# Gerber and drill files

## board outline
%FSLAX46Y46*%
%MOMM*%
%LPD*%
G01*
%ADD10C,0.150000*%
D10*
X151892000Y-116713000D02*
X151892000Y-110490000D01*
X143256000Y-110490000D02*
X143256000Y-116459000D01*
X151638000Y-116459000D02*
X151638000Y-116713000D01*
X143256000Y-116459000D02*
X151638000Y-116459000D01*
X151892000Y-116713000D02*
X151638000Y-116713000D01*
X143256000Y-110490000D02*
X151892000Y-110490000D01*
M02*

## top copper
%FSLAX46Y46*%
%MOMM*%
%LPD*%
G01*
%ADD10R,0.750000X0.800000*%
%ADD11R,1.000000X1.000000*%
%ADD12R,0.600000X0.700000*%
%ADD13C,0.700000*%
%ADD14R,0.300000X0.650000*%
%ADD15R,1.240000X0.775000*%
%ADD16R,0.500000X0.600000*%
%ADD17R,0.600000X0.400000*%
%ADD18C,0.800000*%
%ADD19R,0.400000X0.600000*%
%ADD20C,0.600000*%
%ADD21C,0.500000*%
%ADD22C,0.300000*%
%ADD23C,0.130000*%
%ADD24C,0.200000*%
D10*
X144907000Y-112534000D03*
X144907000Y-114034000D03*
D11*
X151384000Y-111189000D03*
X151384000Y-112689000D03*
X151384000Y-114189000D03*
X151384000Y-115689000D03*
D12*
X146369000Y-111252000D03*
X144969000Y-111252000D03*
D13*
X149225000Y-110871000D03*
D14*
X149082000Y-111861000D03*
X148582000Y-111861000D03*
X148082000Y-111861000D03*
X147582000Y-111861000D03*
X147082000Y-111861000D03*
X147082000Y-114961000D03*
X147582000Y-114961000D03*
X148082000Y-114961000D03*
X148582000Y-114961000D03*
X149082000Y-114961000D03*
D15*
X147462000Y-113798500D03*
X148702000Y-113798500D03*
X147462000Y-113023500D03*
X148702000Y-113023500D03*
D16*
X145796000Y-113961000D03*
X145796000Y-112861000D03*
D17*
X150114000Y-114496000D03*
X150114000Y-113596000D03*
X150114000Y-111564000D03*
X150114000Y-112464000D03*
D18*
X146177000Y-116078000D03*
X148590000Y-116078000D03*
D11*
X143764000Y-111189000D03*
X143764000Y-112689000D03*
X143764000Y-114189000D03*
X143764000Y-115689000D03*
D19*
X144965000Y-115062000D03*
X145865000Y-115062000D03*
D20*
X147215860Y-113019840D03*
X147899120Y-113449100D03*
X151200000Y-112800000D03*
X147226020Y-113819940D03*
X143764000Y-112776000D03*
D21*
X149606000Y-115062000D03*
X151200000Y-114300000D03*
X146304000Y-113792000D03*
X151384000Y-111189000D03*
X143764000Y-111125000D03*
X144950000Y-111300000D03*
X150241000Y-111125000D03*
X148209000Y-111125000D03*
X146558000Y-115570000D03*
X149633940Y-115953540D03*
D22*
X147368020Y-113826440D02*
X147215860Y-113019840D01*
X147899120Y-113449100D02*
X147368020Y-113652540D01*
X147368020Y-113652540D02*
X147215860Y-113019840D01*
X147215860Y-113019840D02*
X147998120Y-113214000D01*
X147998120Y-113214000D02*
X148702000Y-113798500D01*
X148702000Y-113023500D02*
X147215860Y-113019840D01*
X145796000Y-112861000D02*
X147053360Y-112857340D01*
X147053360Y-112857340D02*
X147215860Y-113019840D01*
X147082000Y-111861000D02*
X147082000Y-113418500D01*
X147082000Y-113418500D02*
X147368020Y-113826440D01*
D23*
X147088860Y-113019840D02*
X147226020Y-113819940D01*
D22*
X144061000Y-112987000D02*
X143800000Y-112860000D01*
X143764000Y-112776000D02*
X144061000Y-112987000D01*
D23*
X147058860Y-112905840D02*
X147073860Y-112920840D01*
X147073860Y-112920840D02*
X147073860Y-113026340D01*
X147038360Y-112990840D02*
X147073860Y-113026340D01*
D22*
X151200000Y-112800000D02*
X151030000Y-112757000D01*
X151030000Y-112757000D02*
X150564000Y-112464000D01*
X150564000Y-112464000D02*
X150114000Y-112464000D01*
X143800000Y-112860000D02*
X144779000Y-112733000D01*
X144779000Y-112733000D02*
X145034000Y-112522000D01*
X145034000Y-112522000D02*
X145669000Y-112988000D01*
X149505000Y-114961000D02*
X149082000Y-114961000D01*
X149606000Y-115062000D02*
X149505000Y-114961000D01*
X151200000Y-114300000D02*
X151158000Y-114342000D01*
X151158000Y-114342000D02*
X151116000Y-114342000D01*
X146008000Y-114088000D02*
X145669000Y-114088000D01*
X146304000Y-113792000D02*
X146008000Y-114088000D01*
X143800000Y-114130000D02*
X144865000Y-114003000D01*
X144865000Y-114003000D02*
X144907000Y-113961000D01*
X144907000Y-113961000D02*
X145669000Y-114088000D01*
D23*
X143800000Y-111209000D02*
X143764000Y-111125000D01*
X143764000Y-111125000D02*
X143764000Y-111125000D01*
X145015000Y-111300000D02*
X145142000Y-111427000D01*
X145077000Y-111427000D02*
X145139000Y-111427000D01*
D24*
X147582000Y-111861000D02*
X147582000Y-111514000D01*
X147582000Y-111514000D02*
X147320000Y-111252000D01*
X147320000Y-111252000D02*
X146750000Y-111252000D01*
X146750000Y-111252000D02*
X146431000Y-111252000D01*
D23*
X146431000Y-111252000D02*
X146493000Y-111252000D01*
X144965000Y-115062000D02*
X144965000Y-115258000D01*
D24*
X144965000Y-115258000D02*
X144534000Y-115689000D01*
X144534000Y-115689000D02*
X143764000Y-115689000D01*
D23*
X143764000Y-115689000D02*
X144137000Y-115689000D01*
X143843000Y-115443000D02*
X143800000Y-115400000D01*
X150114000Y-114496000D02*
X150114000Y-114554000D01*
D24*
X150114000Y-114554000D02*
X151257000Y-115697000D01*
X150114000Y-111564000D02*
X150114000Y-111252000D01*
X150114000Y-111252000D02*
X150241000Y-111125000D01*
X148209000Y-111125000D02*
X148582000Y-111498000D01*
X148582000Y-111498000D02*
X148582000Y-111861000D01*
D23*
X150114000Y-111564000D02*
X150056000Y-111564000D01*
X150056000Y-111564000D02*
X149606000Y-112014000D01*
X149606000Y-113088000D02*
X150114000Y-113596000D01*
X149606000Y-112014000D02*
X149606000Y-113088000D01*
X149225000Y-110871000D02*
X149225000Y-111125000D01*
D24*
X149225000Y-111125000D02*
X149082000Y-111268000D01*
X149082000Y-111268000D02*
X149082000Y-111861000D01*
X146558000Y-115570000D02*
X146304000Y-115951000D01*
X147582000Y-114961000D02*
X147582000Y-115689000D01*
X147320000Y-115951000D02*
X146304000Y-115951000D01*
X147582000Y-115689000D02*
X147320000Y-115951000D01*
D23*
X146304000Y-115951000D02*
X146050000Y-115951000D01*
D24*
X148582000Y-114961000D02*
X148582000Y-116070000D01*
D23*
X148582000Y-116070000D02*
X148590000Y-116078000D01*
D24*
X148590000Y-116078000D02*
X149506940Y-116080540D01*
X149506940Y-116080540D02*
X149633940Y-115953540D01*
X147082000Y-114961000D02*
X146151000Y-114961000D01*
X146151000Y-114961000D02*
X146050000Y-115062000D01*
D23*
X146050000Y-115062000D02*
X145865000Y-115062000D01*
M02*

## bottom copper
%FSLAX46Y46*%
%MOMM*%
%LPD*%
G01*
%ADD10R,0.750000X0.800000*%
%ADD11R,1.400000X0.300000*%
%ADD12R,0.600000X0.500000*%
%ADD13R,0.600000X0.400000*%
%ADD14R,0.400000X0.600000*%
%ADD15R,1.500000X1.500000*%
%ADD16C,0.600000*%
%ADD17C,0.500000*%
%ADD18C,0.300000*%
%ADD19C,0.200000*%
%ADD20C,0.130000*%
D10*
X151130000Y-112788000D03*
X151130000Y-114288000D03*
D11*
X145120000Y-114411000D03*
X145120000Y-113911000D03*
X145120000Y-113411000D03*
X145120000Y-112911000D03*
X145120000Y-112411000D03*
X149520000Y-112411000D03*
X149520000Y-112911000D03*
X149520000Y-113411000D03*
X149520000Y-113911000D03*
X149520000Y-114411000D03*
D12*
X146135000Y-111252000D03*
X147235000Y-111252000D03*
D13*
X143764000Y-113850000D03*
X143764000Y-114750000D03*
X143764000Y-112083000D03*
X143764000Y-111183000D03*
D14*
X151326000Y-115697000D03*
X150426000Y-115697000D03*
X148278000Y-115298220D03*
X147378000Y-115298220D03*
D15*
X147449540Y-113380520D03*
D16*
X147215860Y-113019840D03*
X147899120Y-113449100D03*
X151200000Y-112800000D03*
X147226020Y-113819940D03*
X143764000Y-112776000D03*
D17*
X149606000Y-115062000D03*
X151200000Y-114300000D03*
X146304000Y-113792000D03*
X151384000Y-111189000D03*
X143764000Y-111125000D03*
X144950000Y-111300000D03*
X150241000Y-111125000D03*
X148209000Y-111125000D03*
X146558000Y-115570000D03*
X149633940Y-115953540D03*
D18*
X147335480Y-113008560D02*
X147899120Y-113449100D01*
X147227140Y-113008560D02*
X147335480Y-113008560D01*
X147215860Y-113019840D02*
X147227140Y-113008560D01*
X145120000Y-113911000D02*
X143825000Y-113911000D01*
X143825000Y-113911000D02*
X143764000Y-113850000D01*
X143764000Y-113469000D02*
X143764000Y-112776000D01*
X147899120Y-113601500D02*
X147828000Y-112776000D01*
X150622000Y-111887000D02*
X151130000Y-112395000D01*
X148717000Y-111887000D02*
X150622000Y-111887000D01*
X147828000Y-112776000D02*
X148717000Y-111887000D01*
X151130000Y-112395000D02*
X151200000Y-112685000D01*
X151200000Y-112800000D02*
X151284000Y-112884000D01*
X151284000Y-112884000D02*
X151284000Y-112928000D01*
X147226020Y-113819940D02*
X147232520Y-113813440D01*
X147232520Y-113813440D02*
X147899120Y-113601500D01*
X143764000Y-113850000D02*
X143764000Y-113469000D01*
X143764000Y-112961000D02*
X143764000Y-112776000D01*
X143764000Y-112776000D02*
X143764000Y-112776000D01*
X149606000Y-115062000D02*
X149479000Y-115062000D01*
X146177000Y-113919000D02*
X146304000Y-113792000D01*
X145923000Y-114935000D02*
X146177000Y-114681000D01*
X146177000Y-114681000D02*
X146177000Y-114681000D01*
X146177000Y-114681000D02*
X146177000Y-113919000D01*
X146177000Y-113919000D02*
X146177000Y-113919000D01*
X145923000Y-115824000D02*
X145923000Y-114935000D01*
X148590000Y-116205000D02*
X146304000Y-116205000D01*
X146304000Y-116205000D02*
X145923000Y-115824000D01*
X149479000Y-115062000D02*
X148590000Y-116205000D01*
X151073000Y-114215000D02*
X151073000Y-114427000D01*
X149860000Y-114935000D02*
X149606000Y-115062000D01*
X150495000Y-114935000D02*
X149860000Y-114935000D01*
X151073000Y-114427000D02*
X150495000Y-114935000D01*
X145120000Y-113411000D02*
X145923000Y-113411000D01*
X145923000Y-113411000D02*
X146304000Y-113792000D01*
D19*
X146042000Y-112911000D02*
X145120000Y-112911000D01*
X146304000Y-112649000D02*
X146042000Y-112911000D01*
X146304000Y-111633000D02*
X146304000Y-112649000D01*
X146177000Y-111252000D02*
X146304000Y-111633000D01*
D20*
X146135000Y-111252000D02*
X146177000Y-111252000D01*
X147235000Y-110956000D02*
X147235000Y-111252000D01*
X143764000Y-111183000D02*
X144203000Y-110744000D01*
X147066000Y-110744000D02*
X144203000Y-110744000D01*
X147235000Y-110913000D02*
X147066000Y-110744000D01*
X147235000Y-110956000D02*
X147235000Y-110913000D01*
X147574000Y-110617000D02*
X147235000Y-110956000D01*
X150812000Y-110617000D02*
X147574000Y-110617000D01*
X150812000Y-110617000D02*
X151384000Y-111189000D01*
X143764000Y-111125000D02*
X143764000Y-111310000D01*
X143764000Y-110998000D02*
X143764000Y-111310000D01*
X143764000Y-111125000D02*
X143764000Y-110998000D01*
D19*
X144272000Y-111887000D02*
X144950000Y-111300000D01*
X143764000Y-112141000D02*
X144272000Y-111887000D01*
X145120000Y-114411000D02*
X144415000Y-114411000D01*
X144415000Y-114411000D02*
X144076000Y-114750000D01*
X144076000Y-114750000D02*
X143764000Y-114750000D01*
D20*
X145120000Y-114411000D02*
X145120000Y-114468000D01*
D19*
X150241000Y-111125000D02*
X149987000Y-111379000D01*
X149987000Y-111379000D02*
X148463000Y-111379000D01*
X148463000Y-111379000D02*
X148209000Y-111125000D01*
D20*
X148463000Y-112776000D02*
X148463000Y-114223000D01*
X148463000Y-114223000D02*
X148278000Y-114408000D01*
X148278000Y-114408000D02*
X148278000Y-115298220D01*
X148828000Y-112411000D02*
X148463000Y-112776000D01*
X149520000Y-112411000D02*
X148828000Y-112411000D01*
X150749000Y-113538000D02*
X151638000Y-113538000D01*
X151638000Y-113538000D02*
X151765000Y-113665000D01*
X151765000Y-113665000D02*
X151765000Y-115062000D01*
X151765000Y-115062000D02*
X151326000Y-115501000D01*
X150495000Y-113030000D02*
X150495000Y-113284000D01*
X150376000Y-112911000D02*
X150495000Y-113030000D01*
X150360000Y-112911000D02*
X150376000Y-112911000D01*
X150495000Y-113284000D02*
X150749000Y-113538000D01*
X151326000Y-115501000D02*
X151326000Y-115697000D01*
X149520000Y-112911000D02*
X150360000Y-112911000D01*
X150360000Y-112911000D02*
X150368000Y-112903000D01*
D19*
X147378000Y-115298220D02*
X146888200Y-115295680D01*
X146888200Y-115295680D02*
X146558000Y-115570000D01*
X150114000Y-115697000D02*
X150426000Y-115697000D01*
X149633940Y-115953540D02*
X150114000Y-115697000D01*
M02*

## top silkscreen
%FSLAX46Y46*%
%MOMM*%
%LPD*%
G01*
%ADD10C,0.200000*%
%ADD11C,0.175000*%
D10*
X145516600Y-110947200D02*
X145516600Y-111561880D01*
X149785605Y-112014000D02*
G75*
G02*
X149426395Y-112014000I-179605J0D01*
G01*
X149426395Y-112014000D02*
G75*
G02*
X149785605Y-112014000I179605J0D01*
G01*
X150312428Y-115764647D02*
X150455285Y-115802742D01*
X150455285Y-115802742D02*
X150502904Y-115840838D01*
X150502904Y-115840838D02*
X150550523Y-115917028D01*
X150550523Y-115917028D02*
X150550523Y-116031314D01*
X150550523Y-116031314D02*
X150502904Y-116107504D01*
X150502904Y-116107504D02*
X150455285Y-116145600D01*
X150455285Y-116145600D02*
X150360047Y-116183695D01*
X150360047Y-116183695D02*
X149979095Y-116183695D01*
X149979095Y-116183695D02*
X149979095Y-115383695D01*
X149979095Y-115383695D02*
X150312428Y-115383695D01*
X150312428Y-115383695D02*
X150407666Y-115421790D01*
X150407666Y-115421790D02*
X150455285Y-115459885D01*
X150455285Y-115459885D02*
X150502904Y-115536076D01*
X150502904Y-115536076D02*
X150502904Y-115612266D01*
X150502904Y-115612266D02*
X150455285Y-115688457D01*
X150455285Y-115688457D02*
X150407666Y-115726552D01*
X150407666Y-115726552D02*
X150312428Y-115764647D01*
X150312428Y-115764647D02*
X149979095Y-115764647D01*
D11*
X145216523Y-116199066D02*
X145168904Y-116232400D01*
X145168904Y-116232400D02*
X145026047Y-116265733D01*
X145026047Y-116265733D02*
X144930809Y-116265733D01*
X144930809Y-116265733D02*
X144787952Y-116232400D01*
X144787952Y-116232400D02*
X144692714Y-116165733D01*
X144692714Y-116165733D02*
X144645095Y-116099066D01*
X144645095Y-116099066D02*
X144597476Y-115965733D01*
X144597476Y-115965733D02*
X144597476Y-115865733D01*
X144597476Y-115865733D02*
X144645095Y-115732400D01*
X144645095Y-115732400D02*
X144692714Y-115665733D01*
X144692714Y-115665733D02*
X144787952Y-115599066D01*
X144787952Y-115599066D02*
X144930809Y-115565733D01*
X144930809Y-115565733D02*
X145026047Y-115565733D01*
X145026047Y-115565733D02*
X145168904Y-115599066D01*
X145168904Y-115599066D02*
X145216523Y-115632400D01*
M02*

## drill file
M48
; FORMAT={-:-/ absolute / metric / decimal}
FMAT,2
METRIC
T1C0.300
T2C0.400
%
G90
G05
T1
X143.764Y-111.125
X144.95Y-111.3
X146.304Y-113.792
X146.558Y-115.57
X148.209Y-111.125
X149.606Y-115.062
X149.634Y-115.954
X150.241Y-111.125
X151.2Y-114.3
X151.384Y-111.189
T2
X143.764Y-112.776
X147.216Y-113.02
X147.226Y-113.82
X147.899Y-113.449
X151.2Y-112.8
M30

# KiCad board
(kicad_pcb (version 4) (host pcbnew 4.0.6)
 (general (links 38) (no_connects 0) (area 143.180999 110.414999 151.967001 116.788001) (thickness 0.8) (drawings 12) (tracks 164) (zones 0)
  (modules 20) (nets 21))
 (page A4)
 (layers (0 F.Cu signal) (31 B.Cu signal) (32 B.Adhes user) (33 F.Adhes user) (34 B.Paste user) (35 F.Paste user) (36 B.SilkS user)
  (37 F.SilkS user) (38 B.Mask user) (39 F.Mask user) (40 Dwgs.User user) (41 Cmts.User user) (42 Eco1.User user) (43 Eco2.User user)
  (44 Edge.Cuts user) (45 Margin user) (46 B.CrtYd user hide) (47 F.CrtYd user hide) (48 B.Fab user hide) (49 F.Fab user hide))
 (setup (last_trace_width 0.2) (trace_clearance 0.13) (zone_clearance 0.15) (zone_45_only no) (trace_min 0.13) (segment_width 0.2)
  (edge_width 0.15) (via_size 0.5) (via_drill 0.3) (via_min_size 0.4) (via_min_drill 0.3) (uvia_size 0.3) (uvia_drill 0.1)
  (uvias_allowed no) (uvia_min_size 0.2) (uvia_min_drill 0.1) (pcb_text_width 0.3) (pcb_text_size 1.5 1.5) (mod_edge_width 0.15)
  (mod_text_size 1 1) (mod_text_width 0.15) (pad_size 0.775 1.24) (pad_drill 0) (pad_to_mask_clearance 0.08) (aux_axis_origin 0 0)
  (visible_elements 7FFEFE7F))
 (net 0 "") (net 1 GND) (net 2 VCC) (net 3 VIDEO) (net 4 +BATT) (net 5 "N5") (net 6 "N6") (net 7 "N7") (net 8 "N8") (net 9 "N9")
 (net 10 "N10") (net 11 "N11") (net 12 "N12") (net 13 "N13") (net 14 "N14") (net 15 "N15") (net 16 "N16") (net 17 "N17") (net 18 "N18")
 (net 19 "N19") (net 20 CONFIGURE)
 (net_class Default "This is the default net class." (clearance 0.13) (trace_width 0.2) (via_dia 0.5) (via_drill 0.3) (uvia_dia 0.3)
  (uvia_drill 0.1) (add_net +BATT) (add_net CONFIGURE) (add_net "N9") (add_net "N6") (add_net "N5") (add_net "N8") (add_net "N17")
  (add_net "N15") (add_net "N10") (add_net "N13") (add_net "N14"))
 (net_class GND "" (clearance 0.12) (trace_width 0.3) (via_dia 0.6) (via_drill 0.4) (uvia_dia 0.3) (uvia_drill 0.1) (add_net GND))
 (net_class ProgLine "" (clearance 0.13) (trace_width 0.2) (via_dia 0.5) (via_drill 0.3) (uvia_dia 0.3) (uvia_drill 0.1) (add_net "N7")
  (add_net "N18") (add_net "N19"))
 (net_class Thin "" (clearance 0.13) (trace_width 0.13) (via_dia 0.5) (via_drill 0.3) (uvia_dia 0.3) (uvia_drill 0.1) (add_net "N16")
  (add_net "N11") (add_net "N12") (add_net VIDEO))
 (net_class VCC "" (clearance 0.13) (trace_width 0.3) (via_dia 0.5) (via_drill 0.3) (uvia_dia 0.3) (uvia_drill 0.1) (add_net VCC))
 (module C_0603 (layer B.Cu) (at 151.13 113.538 270)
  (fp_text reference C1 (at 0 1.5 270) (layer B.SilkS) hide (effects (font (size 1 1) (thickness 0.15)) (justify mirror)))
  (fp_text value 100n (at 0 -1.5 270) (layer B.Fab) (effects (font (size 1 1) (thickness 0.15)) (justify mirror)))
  (pad 1 smd rect (at -0.75 0 270) (size 0.8 0.75) (layers B.Cu B.Paste B.Mask) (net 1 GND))
  (pad 2 smd rect (at 0.75 0 270) (size 0.8 0.75) (layers B.Cu B.Paste B.Mask) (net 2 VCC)))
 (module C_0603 (layer F.Cu) (at 144.907 113.284 270)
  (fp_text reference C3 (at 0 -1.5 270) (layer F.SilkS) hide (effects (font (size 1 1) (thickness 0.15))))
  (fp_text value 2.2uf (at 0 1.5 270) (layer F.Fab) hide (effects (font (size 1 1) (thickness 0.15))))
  (pad 1 smd rect (at -0.75 0 270) (size 0.8 0.75) (layers F.Cu F.Paste F.Mask) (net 1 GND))
  (pad 2 smd rect (at 0.75 0 270) (size 0.8 0.75) (layers F.Cu F.Paste F.Mask) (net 2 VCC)))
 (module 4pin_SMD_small (layer F.Cu) (at 151.384 115.189 90)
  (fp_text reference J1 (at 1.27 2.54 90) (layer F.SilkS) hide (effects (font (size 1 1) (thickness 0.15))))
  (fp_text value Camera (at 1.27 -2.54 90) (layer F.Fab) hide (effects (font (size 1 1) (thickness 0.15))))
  (pad 4 smd rect (at 4 0 90) (size 1 1) (layers F.Cu F.Paste F.Mask) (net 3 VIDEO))
  (pad 3 smd rect (at 2.5 0 90) (size 1 1) (layers F.Cu F.Paste F.Mask) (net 1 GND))
  (pad 2 smd rect (at 1 0 90) (size 1 1) (layers F.Cu F.Paste F.Mask) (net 2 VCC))
  (pad 1 smd rect (at -0.5 0 90) (size 1 1) (layers F.Cu F.Paste F.Mask) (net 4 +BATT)))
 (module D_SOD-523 (layer F.Cu) (at 145.669 111.252)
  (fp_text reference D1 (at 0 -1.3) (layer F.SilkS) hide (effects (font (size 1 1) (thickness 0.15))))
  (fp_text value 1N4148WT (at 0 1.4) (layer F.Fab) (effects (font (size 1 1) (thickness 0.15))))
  (pad 2 smd rect (at 0.7 0 180) (size 0.6 0.7) (layers F.Cu F.Paste F.Mask) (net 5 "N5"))
  (pad 1 smd rect (at -0.7 0 180) (size 0.6 0.7) (layers F.Cu F.Paste F.Mask) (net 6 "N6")))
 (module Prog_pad (layer F.Cu) (at 149.225 110.871)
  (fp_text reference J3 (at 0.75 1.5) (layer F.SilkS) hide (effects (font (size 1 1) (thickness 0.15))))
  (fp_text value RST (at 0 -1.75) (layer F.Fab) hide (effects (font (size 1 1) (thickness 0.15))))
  (pad 1 smd circle (at 0 0) (size 0.7 0.7) (layers F.Cu F.Paste F.Mask) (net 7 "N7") (solder_mask_margin 0.02)))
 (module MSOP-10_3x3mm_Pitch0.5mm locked (layer B.Cu) (at 147.32 113.411)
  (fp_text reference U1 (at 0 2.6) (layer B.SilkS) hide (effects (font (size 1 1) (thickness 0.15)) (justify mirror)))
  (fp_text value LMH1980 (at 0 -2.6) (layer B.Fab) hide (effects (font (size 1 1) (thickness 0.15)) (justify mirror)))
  (pad 1 smd rect (at -2.2 1) (size 1.4 0.3) (layers B.Cu B.Paste B.Mask) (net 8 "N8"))
  (pad 2 smd rect (at -2.2 0.5) (size 1.4 0.3) (layers B.Cu B.Paste B.Mask) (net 1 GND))
  (pad 3 smd rect (at -2.2 0) (size 1.4 0.3) (layers B.Cu B.Paste B.Mask) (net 2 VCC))
  (pad 4 smd rect (at -2.2 -0.5) (size 1.4 0.3) (layers B.Cu B.Paste B.Mask) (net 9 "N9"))
  (pad 5 smd rect (at -2.2 -1) (size 1.4 0.3) (layers B.Cu B.Paste B.Mask) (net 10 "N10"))
  (pad 6 smd rect (at 2.2 -1) (size 1.4 0.3) (layers B.Cu B.Paste B.Mask) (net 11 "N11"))
  (pad 7 smd rect (at 2.2 -0.5) (size 1.4 0.3) (layers B.Cu B.Paste B.Mask) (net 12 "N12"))
  (pad 8 smd rect (at 2.2 0) (size 1.4 0.3) (layers B.Cu B.Paste B.Mask) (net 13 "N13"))
  (pad 9 smd rect (at 2.2 0.5) (size 1.4 0.3) (layers B.Cu B.Paste B.Mask) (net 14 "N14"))
  (pad 10 smd rect (at 2.2 1) (size 1.4 0.3) (layers B.Cu B.Paste B.Mask) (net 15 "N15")))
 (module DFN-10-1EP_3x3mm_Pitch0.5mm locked (layer F.Cu) (at 148.082 113.411 270)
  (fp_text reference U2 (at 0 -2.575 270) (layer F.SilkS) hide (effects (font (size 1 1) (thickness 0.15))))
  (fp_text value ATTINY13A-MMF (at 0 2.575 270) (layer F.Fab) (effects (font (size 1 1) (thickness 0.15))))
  (pad 1 smd rect (at -1.55 -1 270) (size 0.65 0.3) (layers F.Cu F.Paste F.Mask) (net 7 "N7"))
  (pad 2 smd rect (at -1.55 -0.5 270) (size 0.65 0.3) (layers F.Cu F.Paste F.Mask) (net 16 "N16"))
  (pad 3 smd rect (at -1.55 0 270) (size 0.65 0.3) (layers F.Cu F.Paste F.Mask))
  (pad 4 smd rect (at -1.55 0.5 270) (size 0.65 0.3) (layers F.Cu F.Paste F.Mask) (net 5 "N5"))
  (pad 5 smd rect (at -1.55 1 270) (size 0.65 0.3) (layers F.Cu F.Paste F.Mask) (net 1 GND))
  (pad 6 smd rect (at 1.55 1 270) (size 0.65 0.3) (layers F.Cu F.Paste F.Mask) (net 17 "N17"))
  (pad 7 smd rect (at 1.55 0.5 270) (size 0.65 0.3) (layers F.Cu F.Paste F.Mask) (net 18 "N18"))
  (pad 8 smd rect (at 1.55 0 270) (size 0.65 0.3) (layers F.Cu F.Paste F.Mask))
  (pad 9 smd rect (at 1.55 -0.5 270) (size 0.65 0.3) (layers F.Cu F.Paste F.Mask) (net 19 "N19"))
  (pad 10 smd rect (at 1.55 -1 270) (size 0.65 0.3) (layers F.Cu F.Paste F.Mask) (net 2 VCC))
  (pad 11 smd rect (at 0.3875 0.62 270) (size 0.775 1.24) (layers F.Cu F.Paste F.Mask) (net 1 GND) (solder_paste_margin_ratio -0.2))
  (pad 11 smd rect (at 0.3875 -0.62 270) (size 0.775 1.24) (layers F.Cu F.Paste F.Mask) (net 1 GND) (solder_paste_margin_ratio -0.2))
  (pad 11 smd rect (at -0.3875 0.62 270) (size 0.775 1.24) (layers F.Cu F.Paste F.Mask) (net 1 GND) (solder_paste_margin_ratio -0.2))
  (pad 11 smd rect (at -0.3875 -0.62 270) (size 0.775 1.24) (layers F.Cu F.Paste F.Mask) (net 1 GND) (solder_paste_margin_ratio -0.2)))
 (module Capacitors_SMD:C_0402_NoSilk (layer B.Cu) (at 146.685 111.252)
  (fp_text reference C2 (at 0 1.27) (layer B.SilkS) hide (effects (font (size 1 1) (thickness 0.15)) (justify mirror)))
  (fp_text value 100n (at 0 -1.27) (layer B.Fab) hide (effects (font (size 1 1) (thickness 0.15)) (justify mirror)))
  (pad 1 smd rect (at -0.55 0) (size 0.6 0.5) (layers B.Cu B.Paste B.Mask) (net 9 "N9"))
  (pad 2 smd rect (at 0.55 0) (size 0.6 0.5) (layers B.Cu B.Paste B.Mask) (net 3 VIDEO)))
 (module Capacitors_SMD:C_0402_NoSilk (layer F.Cu) (at 145.796 113.411 90)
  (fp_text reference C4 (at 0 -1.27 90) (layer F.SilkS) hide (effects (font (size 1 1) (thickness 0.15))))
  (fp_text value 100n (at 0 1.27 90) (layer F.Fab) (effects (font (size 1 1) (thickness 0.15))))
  (pad 1 smd rect (at -0.55 0 90) (size 0.6 0.5) (layers F.Cu F.Paste F.Mask) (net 2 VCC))
  (pad 2 smd rect (at 0.55 0 90) (size 0.6 0.5) (layers F.Cu F.Paste F.Mask) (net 1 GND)))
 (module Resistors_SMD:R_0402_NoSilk (layer B.Cu) (at 143.764 114.3 270)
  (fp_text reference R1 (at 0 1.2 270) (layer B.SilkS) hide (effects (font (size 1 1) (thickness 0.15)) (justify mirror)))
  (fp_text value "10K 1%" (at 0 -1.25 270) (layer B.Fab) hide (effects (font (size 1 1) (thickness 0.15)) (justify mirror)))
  (pad 1 smd rect (at -0.45 0 270) (size 0.4 0.6) (layers B.Cu B.Paste B.Mask) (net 1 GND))
  (pad 2 smd rect (at 0.45 0 270) (size 0.4 0.6) (layers B.Cu B.Paste B.Mask) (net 8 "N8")))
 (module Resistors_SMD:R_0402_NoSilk (layer B.Cu) (at 143.764 111.633 90)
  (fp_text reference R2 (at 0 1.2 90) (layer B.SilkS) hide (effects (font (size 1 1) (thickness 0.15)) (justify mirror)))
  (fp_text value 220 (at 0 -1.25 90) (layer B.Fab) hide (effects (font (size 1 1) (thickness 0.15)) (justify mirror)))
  (pad 1 smd rect (at -0.45 0 90) (size 0.4 0.6) (layers B.Cu B.Paste B.Mask) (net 6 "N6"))
  (pad 2 smd rect (at 0.45 0 90) (size 0.4 0.6) (layers B.Cu B.Paste B.Mask) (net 3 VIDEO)))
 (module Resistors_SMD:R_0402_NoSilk (layer F.Cu) (at 150.114 114.046 90)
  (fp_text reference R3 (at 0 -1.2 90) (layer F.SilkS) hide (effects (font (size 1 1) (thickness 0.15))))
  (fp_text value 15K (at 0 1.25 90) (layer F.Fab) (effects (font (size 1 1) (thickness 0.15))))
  (pad 1 smd rect (at -0.45 0 90) (size 0.4 0.6) (layers F.Cu F.Paste F.Mask) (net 4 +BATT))
  (pad 2 smd rect (at 0.45 0 90) (size 0.4 0.6) (layers F.Cu F.Paste F.Mask) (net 16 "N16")))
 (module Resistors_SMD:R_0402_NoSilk (layer F.Cu) (at 150.114 112.014 270)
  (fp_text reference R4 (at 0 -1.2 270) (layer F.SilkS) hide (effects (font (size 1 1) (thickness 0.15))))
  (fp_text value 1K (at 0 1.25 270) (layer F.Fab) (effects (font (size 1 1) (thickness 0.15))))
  (pad 1 smd rect (at -0.45 0 270) (size 0.4 0.6) (layers F.Cu F.Paste F.Mask) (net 16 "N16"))
  (pad 2 smd rect (at 0.45 0 270) (size 0.4 0.6) (layers F.Cu F.Paste F.Mask) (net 1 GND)))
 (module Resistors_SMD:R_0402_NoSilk (layer B.Cu) (at 150.876 115.697 180)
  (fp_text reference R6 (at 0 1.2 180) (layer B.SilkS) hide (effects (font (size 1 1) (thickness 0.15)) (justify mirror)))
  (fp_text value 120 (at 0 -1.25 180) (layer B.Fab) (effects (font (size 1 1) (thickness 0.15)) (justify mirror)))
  (pad 1 smd rect (at -0.45 0 180) (size 0.4 0.6) (layers B.Cu B.Paste B.Mask) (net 12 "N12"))
  (pad 2 smd rect (at 0.45 0 180) (size 0.4 0.6) (layers B.Cu B.Paste B.Mask) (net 19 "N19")))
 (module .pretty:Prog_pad (layer F.Cu) (at 146.177 116.078)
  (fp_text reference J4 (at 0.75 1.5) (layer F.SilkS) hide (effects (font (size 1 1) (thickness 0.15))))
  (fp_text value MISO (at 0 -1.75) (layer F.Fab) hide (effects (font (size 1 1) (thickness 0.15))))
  (pad 1 smd circle (at 0 0) (size 0.8 0.8) (layers F.Cu F.Paste F.Mask) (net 18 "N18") (solder_mask_margin 0.02)))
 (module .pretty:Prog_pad (layer F.Cu) (at 148.59 116.078)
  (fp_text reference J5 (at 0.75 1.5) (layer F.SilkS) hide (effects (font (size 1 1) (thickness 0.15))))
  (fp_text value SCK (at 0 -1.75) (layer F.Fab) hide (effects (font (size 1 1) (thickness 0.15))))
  (pad 1 smd circle (at 0 0) (size 0.8 0.8) (layers F.Cu F.Paste F.Mask) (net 19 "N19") (solder_mask_margin 0.02)))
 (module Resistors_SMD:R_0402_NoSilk (layer B.Cu) (at 147.828 115.29822 180)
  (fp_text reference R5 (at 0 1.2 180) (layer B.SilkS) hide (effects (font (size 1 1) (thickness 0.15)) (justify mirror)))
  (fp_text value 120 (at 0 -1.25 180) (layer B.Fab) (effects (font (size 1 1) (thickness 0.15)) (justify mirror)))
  (pad 1 smd rect (at -0.45 0 180) (size 0.4 0.6) (layers B.Cu B.Paste B.Mask) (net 11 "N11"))
  (pad 2 smd rect (at 0.45 0 180) (size 0.4 0.6) (layers B.Cu B.Paste B.Mask) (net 18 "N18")))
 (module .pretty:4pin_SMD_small (layer F.Cu) (at 143.764 115.189 90)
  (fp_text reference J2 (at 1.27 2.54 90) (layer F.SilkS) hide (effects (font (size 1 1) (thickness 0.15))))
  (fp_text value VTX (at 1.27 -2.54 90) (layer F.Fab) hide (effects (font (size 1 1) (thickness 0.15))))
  (pad 4 smd rect (at 4 0 90) (size 1 1) (layers F.Cu F.Paste F.Mask) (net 3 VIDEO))
  (pad 3 smd rect (at 2.5 0 90) (size 1 1) (layers F.Cu F.Paste F.Mask) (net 1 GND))
  (pad 2 smd rect (at 1 0 90) (size 1 1) (layers F.Cu F.Paste F.Mask) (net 2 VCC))
  (pad 1 smd rect (at -0.5 0 90) (size 1 1) (layers F.Cu F.Paste F.Mask) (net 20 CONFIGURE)))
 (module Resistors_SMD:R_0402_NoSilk (layer F.Cu) (at 145.415 115.062)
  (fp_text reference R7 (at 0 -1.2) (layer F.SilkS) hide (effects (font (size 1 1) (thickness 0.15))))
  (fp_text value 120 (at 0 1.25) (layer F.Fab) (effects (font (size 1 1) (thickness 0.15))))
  (pad 1 smd rect (at -0.45 0) (size 0.4 0.6) (layers F.Cu F.Paste F.Mask) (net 20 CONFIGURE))
  (pad 2 smd rect (at 0.45 0) (size 0.4 0.6) (layers F.Cu F.Paste F.Mask) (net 17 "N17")))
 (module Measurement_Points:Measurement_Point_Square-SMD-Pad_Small (layer B.Cu) (at 147.44954 113.38052)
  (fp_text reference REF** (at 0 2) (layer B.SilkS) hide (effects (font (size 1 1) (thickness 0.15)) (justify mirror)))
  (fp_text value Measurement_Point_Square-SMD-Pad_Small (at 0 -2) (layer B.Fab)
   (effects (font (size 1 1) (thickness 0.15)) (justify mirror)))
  (pad 1 smd rect (at 0 0) (size 1.5 1.5) (layers B.Cu B.Mask) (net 1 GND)))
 (gr_line (start 145.5166 110.9472) (end 145.5166 111.56188) (angle 90) (layer F.SilkS) (width 0.2))
 (gr_line (start 151.892 116.713) (end 151.892 110.49) (angle 90) (layer Edge.Cuts) (width 0.15))
 (gr_line (start 143.256 110.49) (end 143.256 116.459) (angle 90) (layer Edge.Cuts) (width 0.15))
 (gr_line (start 151.638 116.459) (end 151.638 116.713) (angle 90) (layer Edge.Cuts) (width 0.15))
 (gr_line (start 143.256 116.459) (end 151.638 116.459) (angle 90) (layer Edge.Cuts) (width 0.15))
 (gr_line (start 151.892 116.713) (end 151.638 116.713) (angle 90) (layer Edge.Cuts) (width 0.15))
 (gr_circle (center 149.606 112.014) (end 149.479 111.887) (layer F.SilkS) (width 0.2))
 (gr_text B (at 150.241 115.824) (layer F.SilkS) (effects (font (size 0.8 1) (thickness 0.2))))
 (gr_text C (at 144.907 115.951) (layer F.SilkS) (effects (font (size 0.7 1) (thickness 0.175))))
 (gr_line (start 143.256 110.49) (end 151.892 110.49) (angle 90) (layer Edge.Cuts) (width 0.15))
 (segment (start 147.36802 113.82644) (end 147.21586 113.01984) (width 0.3) (layer F.Cu) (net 1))
 (via (at 147.21586 113.01984) (size 0.6) (drill 0.4) (layers F.Cu B.Cu) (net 1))
 (segment (start 147.89912 113.4491) (end 147.36802 113.65254) (width 0.3) (layer F.Cu) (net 1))
 (via (at 147.89912 113.4491) (size 0.6) (drill 0.4) (layers F.Cu B.Cu) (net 1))
 (segment (start 147.33548 113.00856) (end 147.89912 113.4491) (width 0.3) (layer B.Cu) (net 1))
 (segment (start 147.22714 113.00856) (end 147.33548 113.00856) (width 0.3) (layer B.Cu) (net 1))
 (segment (start 147.21586 113.01984) (end 147.22714 113.00856) (width 0.3) (layer B.Cu) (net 1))
 (segment (start 147.36802 113.65254) (end 147.21586 113.01984) (width 0.3) (layer F.Cu) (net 1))
 (segment (start 147.21586 113.01984) (end 147.99812 113.214) (width 0.3) (layer F.Cu) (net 1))
 (segment (start 147.99812 113.214) (end 148.702 113.7985) (width 0.3) (layer F.Cu) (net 1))
 (segment (start 148.702 113.0235) (end 147.21586 113.01984) (width 0.3) (layer F.Cu) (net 1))
 (segment (start 145.796 112.861) (end 147.05336 112.85734) (width 0.3) (layer F.Cu) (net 1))
 (segment (start 147.05336 112.85734) (end 147.21586 113.01984) (width 0.3) (layer F.Cu) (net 1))
 (segment (start 147.082 111.861) (end 147.082 113.4185) (width 0.3) (layer F.Cu) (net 1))
 (segment (start 147.082 113.4185) (end 147.36802 113.82644) (width 0.3) (layer F.Cu) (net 1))
 (segment (start 145.12 113.911) (end 143.825 113.911) (width 0.3) (layer B.Cu) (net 1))
 (segment (start 143.825 113.911) (end 143.764 113.85) (width 0.3) (layer B.Cu) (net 1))
 (segment (start 143.764 113.469) (end 143.764 112.776) (width 0.3) (layer B.Cu) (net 1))
 (segment (start 147.89912 113.6015) (end 147.828 112.776) (width 0.3) (layer B.Cu) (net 1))
 (segment (start 150.622 111.887) (end 151.13 112.395) (width 0.3) (layer B.Cu) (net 1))
 (segment (start 148.717 111.887) (end 150.622 111.887) (width 0.3) (layer B.Cu) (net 1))
 (segment (start 147.828 112.776) (end 148.717 111.887) (width 0.3) (layer B.Cu) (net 1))
 (segment (start 151.13 112.395) (end 151.2 112.685) (width 0.3) (layer B.Cu) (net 1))
 (via (at 151.2 112.8) (size 0.6) (drill 0.4) (layers F.Cu B.Cu) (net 1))
 (segment (start 151.2 112.8) (end 151.284 112.884) (width 0.3) (layer B.Cu) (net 1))
 (segment (start 151.284 112.884) (end 151.284 112.928) (width 0.3) (layer B.Cu) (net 1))
 (segment (start 147.08886 113.01984) (end 147.22602 113.81994) (width 0.13) (layer F.Cu) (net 1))
 (via (at 147.22602 113.81994) (size 0.6) (drill 0.4) (layers F.Cu B.Cu) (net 1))
 (segment (start 147.22602 113.81994) (end 147.23252 113.81344) (width 0.3) (layer B.Cu) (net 1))
 (segment (start 147.23252 113.81344) (end 147.89912 113.6015) (width 0.3) (layer B.Cu) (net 1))
 (segment (start 143.764 113.85) (end 143.764 113.469) (width 0.3) (layer B.Cu) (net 1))
 (segment (start 143.764 112.961) (end 143.764 112.776) (width 0.3) (layer B.Cu) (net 1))
 (segment (start 144.061 112.987) (end 143.8 112.86) (width 0.3) (layer F.Cu) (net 1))
 (segment (start 143.764 112.776) (end 144.061 112.987) (width 0.3) (layer F.Cu) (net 1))
 (via (at 143.764 112.776) (size 0.6) (drill 0.4) (layers F.Cu B.Cu) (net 1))
 (segment (start 143.764 112.776) (end 143.764 112.776) (width 0.3) (layer B.Cu) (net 1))
 (segment (start 147.05886 112.90584) (end 147.07386 112.92084) (width 0.13) (layer F.Cu) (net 1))
 (segment (start 147.07386 112.92084) (end 147.07386 113.02634) (width 0.13) (layer F.Cu) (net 1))
 (segment (start 147.03836 112.99084) (end 147.07386 113.02634) (width 0.13) (layer F.Cu) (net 1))
 (segment (start 151.2 112.8) (end 151.03 112.757) (width 0.3) (layer F.Cu) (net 1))
 (segment (start 151.03 112.757) (end 150.564 112.464) (width 0.3) (layer F.Cu) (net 1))
 (segment (start 150.564 112.464) (end 150.114 112.464) (width 0.3) (layer F.Cu) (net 1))
 (segment (start 143.8 112.86) (end 144.779 112.733) (width 0.3) (layer F.Cu) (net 1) (status 20))
 (segment (start 144.779 112.733) (end 145.034 112.522) (width 0.3) (layer F.Cu) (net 1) (status 30))
 (segment (start 145.034 112.522) (end 145.669 112.988) (width 0.3) (layer F.Cu) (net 1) (status 10))
 (segment (start 149.606 115.062) (end 149.479 115.062) (width 0.3) (layer B.Cu) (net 2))
 (segment (start 146.177 113.919) (end 146.304 113.792) (width 0.3) (layer B.Cu) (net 2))
 (segment (start 145.923 114.935) (end 146.177 114.681) (width 0.3) (layer B.Cu) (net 2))
 (segment (start 146.177 114.681) (end 146.177 114.681) (width 0.3) (layer B.Cu) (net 2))
 (segment (start 146.177 114.681) (end 146.177 113.919) (width 0.3) (layer B.Cu) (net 2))
 (segment (start 146.177 113.919) (end 146.177 113.919) (width 0.3) (layer B.Cu) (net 2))
 (segment (start 145.923 115.824) (end 145.923 114.935) (width 0.3) (layer B.Cu) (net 2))
 (segment (start 148.59 116.205) (end 146.304 116.205) (width 0.3) (layer B.Cu) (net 2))
 (segment (start 146.304 116.205) (end 145.923 115.824) (width 0.3) (layer B.Cu) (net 2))
 (segment (start 149.479 115.062) (end 148.59 116.205) (width 0.3) (layer B.Cu) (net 2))
 (segment (start 151.073 114.215) (end 151.073 114.427) (width 0.3) (layer B.Cu) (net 2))
 (segment (start 149.505 114.961) (end 149.082 114.961) (width 0.3) (layer F.Cu) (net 2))
 (segment (start 149.606 115.062) (end 149.505 114.961) (width 0.3) (layer F.Cu) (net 2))
 (via (at 149.606 115.062) (size 0.5) (drill 0.3) (layers F.Cu B.Cu) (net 2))
 (segment (start 149.86 114.935) (end 149.606 115.062) (width 0.3) (layer B.Cu) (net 2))
 (segment (start 150.495 114.935) (end 149.86 114.935) (width 0.3) (layer B.Cu) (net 2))
 (segment (start 151.073 114.427) (end 150.495 114.935) (width 0.3) (layer B.Cu) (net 2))
 (via (at 151.2 114.3) (size 0.5) (drill 0.3) (layers F.Cu B.Cu) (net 2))
 (segment (start 151.2 114.3) (end 151.158 114.342) (width 0.3) (layer F.Cu) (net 2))
 (segment (start 151.158 114.342) (end 151.116 114.342) (width 0.3) (layer F.Cu) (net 2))
 (segment (start 145.12 113.411) (end 145.923 113.411) (width 0.3) (layer B.Cu) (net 2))
 (segment (start 145.923 113.411) (end 146.304 113.792) (width 0.3) (layer B.Cu) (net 2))
 (segment (start 146.008 114.088) (end 145.669 114.088) (width 0.3) (layer F.Cu) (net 2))
 (segment (start 146.304 113.792) (end 146.008 114.088) (width 0.3) (layer F.Cu) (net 2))
 (via (at 146.304 113.792) (size 0.5) (drill 0.3) (layers F.Cu B.Cu) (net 2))
 (segment (start 143.8 114.13) (end 144.865 114.003) (width 0.3) (layer F.Cu) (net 2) (status 20))
 (segment (start 144.865 114.003) (end 144.907 113.961) (width 0.3) (layer F.Cu) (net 2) (status 30))
 (segment (start 144.907 113.961) (end 145.669 114.088) (width 0.3) (layer F.Cu) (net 2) (status 10))
 (segment (start 146.042 112.911) (end 145.12 112.911) (width 0.2) (layer B.Cu) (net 9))
 (segment (start 146.304 112.649) (end 146.042 112.911) (width 0.2) (layer B.Cu) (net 9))
 (segment (start 146.304 111.633) (end 146.304 112.649) (width 0.2) (layer B.Cu) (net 9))
 (segment (start 146.177 111.252) (end 146.304 111.633) (width 0.2) (layer B.Cu) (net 9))
 (segment (start 146.135 111.252) (end 146.177 111.252) (width 0.13) (layer B.Cu) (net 9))
 (segment (start 147.235 110.956) (end 147.235 111.252) (width 0.13) (layer B.Cu) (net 3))
 (via (at 151.384 111.189) (size 0.5) (drill 0.3) (layers F.Cu B.Cu) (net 3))
 (segment (start 143.764 111.183) (end 144.203 110.744) (width 0.13) (layer B.Cu) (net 3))
 (segment (start 147.066 110.744) (end 144.203 110.744) (width 0.13) (layer B.Cu) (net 3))
 (segment (start 147.235 110.913) (end 147.066 110.744) (width 0.13) (layer B.Cu) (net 3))
 (segment (start 147.235 110.956) (end 147.235 110.913) (width 0.13) (layer B.Cu) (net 3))
 (segment (start 147.574 110.617) (end 147.235 110.956) (width 0.13) (layer B.Cu) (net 3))
 (segment (start 150.812 110.617) (end 147.574 110.617) (width 0.13) (layer B.Cu) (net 3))
 (segment (start 150.812 110.617) (end 151.384 111.189) (width 0.13) (layer B.Cu) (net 3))
 (segment (start 143.764 111.125) (end 143.764 111.31) (width 0.13) (layer B.Cu) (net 3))
 (segment (start 143.8 111.209) (end 143.764 111.125) (width 0.13) (layer F.Cu) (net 3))
 (segment (start 143.764 110.998) (end 143.764 111.31) (width 0.13) (layer B.Cu) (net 3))
 (segment (start 143.764 111.125) (end 143.764 110.998) (width 0.13) (layer B.Cu) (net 3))
 (via (at 143.764 111.125) (size 0.5) (drill 0.3) (layers F.Cu B.Cu) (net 3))
 (segment (start 143.764 111.125) (end 143.764 111.125) (width 0.13) (layer F.Cu) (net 3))
 (via (at 144.95 111.3) (size 0.5) (drill 0.3) (layers F.Cu B.Cu) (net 6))
 (segment (start 144.272 111.887) (end 144.95 111.3) (width 0.2) (layer B.Cu) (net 6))
 (segment (start 143.764 112.141) (end 144.272 111.887) (width 0.2) (layer B.Cu) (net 6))
 (segment (start 145.015 111.3) (end 145.142 111.427) (width 0.13) (layer F.Cu) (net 6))
 (segment (start 145.077 111.427) (end 145.139 111.427) (width 0.13) (layer F.Cu) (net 6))
 (segment (start 147.582 111.861) (end 147.582 111.514) (width 0.2) (layer F.Cu) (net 5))
 (segment (start 147.582 111.514) (end 147.32 111.252) (width 0.2) (layer F.Cu) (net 5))
 (segment (start 147.32 111.252) (end 146.75 111.252) (width 0.2) (layer F.Cu) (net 5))
 (segment (start 146.75 111.252) (end 146.431 111.252) (width 0.2) (layer F.Cu) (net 5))
 (segment (start 146.431 111.252) (end 146.493 111.252) (width 0.13) (layer F.Cu) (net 5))
 (segment (start 144.965 115.062) (end 144.965 115.258) (width 0.13) (layer F.Cu) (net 20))
 (segment (start 144.965 115.258) (end 144.534 115.689) (width 0.2) (layer F.Cu) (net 20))
 (segment (start 144.534 115.689) (end 143.764 115.689) (width 0.2) (layer F.Cu) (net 20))
 (segment (start 143.764 115.689) (end 144.137 115.689) (width 0.13) (layer F.Cu) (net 20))
 (segment (start 143.843 115.443) (end 143.8 115.4) (width 0.13) (layer F.Cu) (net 20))
 (segment (start 150.114 114.496) (end 150.114 114.554) (width 0.13) (layer F.Cu) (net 4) (status 10))
 (segment (start 150.114 114.554) (end 151.257 115.697) (width 0.2) (layer F.Cu) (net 4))
 (segment (start 145.12 114.411) (end 144.415 114.411) (width 0.2) (layer B.Cu) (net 8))
 (segment (start 144.415 114.411) (end 144.076 114.75) (width 0.2) (layer B.Cu) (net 8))
 (segment (start 144.076 114.75) (end 143.764 114.75) (width 0.2) (layer B.Cu) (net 8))
 (segment (start 145.12 114.411) (end 145.12 114.468) (width 0.13) (layer B.Cu) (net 8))
 (segment (start 150.114 111.564) (end 150.114 111.252) (width 0.2) (layer F.Cu) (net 16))
 (segment (start 150.114 111.252) (end 150.241 111.125) (width 0.2) (layer F.Cu) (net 16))
 (via (at 150.241 111.125) (size 0.5) (drill 0.3) (layers F.Cu B.Cu) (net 16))
 (segment (start 150.241 111.125) (end 149.987 111.379) (width 0.2) (layer B.Cu) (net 16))
 (segment (start 149.987 111.379) (end 148.463 111.379) (width 0.2) (layer B.Cu) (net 16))
 (segment (start 148.463 111.379) (end 148.209 111.125) (width 0.2) (layer B.Cu) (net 16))
 (via (at 148.209 111.125) (size 0.5) (drill 0.3) (layers F.Cu B.Cu) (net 16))
 (segment (start 148.209 111.125) (end 148.582 111.498) (width 0.2) (layer F.Cu) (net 16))
 (segment (start 148.582 111.498) (end 148.582 111.861) (width 0.2) (layer F.Cu) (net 16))
 (segment (start 150.114 111.564) (end 150.056 111.564) (width 0.13) (layer F.Cu) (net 16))
 (segment (start 150.056 111.564) (end 149.606 112.014) (width 0.13) (layer F.Cu) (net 16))
 (segment (start 149.606 113.088) (end 150.114 113.596) (width 0.13) (layer F.Cu) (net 16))
 (segment (start 149.606 112.014) (end 149.606 113.088) (width 0.13) (layer F.Cu) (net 16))
 (segment (start 148.463 112.776) (end 148.463 114.223) (width 0.13) (layer B.Cu) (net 11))
 (segment (start 148.463 114.223) (end 148.278 114.408) (width 0.13) (layer B.Cu) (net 11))
 (segment (start 148.278 114.408) (end 148.278 115.29822) (width 0.13) (layer B.Cu) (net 11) (status 20))
 (segment (start 148.828 112.411) (end 148.463 112.776) (width 0.13) (layer B.Cu) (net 11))
 (segment (start 149.52 112.411) (end 148.828 112.411) (width 0.13) (layer B.Cu) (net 11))
 (segment (start 150.749 113.538) (end 151.638 113.538) (width 0.13) (layer B.Cu) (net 12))
 (segment (start 151.638 113.538) (end 151.765 113.665) (width 0.13) (layer B.Cu) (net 12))
 (segment (start 151.765 113.665) (end 151.765 115.062) (width 0.13) (layer B.Cu) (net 12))
 (segment (start 151.765 115.062) (end 151.326 115.501) (width 0.13) (layer B.Cu) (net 12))
 (segment (start 150.495 113.03) (end 150.495 113.284) (width 0.13) (layer B.Cu) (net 12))
 (segment (start 150.376 112.911) (end 150.495 113.03) (width 0.13) (layer B.Cu) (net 12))
 (segment (start 150.36 112.911) (end 150.376 112.911) (width 0.13) (layer B.Cu) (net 12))
 (segment (start 150.495 113.284) (end 150.749 113.538) (width 0.13) (layer B.Cu) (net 12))
 (segment (start 151.326 115.501) (end 151.326 115.697) (width 0.13) (layer B.Cu) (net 12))
 (segment (start 149.52 112.911) (end 150.36 112.911) (width 0.13) (layer B.Cu) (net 12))
 (segment (start 150.36 112.911) (end 150.368 112.903) (width 0.13) (layer B.Cu) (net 12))
 (segment (start 149.225 110.871) (end 149.225 111.125) (width 0.13) (layer F.Cu) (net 7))
 (segment (start 149.225 111.125) (end 149.082 111.268) (width 0.2) (layer F.Cu) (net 7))
 (segment (start 149.082 111.268) (end 149.082 111.861) (width 0.2) (layer F.Cu) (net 7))
 (segment (start 147.378 115.29822) (end 146.8882 115.29568) (width 0.2) (layer B.Cu) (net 18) (status 400010))
 (segment (start 146.8882 115.29568) (end 146.558 115.57) (width 0.2) (layer B.Cu) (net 18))
 (via (at 146.558 115.57) (size 0.5) (drill 0.3) (layers F.Cu B.Cu) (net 18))
 (segment (start 146.558 115.57) (end 146.304 115.951) (width 0.2) (layer F.Cu) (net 18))
 (segment (start 147.582 114.961) (end 147.582 115.689) (width 0.2) (layer F.Cu) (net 18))
 (segment (start 147.32 115.951) (end 146.304 115.951) (width 0.2) (layer F.Cu) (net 18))
 (segment (start 147.582 115.689) (end 147.32 115.951) (width 0.2) (layer F.Cu) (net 18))
 (segment (start 146.304 115.951) (end 146.05 115.951) (width 0.13) (layer F.Cu) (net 18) (status 20))
 (segment (start 148.582 114.961) (end 148.582 116.07) (width 0.2) (layer F.Cu) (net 19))
 (segment (start 148.582 116.07) (end 148.59 116.078) (width 0.13) (layer F.Cu) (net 19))
 (segment (start 148.59 116.078) (end 149.50694 116.08054) (width 0.2) (layer F.Cu) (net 19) (status 400000))
 (segment (start 150.114 115.697) (end 150.426 115.697) (width 0.2) (layer B.Cu) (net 19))
 (segment (start 149.63394 115.95354) (end 150.114 115.697) (width 0.2) (layer B.Cu) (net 19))
 (via (at 149.63394 115.95354) (size 0.5) (drill 0.3) (layers F.Cu B.Cu) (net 19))
 (segment (start 149.50694 116.08054) (end 149.63394 115.95354) (width 0.2) (layer F.Cu) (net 19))
 (segment (start 147.082 114.961) (end 146.151 114.961) (width 0.2) (layer F.Cu) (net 17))
 (segment (start 146.151 114.961) (end 146.05 115.062) (width 0.2) (layer F.Cu) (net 17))
 (segment (start 146.05 115.062) (end 145.865 115.062) (width 0.13) (layer F.Cu) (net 17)))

